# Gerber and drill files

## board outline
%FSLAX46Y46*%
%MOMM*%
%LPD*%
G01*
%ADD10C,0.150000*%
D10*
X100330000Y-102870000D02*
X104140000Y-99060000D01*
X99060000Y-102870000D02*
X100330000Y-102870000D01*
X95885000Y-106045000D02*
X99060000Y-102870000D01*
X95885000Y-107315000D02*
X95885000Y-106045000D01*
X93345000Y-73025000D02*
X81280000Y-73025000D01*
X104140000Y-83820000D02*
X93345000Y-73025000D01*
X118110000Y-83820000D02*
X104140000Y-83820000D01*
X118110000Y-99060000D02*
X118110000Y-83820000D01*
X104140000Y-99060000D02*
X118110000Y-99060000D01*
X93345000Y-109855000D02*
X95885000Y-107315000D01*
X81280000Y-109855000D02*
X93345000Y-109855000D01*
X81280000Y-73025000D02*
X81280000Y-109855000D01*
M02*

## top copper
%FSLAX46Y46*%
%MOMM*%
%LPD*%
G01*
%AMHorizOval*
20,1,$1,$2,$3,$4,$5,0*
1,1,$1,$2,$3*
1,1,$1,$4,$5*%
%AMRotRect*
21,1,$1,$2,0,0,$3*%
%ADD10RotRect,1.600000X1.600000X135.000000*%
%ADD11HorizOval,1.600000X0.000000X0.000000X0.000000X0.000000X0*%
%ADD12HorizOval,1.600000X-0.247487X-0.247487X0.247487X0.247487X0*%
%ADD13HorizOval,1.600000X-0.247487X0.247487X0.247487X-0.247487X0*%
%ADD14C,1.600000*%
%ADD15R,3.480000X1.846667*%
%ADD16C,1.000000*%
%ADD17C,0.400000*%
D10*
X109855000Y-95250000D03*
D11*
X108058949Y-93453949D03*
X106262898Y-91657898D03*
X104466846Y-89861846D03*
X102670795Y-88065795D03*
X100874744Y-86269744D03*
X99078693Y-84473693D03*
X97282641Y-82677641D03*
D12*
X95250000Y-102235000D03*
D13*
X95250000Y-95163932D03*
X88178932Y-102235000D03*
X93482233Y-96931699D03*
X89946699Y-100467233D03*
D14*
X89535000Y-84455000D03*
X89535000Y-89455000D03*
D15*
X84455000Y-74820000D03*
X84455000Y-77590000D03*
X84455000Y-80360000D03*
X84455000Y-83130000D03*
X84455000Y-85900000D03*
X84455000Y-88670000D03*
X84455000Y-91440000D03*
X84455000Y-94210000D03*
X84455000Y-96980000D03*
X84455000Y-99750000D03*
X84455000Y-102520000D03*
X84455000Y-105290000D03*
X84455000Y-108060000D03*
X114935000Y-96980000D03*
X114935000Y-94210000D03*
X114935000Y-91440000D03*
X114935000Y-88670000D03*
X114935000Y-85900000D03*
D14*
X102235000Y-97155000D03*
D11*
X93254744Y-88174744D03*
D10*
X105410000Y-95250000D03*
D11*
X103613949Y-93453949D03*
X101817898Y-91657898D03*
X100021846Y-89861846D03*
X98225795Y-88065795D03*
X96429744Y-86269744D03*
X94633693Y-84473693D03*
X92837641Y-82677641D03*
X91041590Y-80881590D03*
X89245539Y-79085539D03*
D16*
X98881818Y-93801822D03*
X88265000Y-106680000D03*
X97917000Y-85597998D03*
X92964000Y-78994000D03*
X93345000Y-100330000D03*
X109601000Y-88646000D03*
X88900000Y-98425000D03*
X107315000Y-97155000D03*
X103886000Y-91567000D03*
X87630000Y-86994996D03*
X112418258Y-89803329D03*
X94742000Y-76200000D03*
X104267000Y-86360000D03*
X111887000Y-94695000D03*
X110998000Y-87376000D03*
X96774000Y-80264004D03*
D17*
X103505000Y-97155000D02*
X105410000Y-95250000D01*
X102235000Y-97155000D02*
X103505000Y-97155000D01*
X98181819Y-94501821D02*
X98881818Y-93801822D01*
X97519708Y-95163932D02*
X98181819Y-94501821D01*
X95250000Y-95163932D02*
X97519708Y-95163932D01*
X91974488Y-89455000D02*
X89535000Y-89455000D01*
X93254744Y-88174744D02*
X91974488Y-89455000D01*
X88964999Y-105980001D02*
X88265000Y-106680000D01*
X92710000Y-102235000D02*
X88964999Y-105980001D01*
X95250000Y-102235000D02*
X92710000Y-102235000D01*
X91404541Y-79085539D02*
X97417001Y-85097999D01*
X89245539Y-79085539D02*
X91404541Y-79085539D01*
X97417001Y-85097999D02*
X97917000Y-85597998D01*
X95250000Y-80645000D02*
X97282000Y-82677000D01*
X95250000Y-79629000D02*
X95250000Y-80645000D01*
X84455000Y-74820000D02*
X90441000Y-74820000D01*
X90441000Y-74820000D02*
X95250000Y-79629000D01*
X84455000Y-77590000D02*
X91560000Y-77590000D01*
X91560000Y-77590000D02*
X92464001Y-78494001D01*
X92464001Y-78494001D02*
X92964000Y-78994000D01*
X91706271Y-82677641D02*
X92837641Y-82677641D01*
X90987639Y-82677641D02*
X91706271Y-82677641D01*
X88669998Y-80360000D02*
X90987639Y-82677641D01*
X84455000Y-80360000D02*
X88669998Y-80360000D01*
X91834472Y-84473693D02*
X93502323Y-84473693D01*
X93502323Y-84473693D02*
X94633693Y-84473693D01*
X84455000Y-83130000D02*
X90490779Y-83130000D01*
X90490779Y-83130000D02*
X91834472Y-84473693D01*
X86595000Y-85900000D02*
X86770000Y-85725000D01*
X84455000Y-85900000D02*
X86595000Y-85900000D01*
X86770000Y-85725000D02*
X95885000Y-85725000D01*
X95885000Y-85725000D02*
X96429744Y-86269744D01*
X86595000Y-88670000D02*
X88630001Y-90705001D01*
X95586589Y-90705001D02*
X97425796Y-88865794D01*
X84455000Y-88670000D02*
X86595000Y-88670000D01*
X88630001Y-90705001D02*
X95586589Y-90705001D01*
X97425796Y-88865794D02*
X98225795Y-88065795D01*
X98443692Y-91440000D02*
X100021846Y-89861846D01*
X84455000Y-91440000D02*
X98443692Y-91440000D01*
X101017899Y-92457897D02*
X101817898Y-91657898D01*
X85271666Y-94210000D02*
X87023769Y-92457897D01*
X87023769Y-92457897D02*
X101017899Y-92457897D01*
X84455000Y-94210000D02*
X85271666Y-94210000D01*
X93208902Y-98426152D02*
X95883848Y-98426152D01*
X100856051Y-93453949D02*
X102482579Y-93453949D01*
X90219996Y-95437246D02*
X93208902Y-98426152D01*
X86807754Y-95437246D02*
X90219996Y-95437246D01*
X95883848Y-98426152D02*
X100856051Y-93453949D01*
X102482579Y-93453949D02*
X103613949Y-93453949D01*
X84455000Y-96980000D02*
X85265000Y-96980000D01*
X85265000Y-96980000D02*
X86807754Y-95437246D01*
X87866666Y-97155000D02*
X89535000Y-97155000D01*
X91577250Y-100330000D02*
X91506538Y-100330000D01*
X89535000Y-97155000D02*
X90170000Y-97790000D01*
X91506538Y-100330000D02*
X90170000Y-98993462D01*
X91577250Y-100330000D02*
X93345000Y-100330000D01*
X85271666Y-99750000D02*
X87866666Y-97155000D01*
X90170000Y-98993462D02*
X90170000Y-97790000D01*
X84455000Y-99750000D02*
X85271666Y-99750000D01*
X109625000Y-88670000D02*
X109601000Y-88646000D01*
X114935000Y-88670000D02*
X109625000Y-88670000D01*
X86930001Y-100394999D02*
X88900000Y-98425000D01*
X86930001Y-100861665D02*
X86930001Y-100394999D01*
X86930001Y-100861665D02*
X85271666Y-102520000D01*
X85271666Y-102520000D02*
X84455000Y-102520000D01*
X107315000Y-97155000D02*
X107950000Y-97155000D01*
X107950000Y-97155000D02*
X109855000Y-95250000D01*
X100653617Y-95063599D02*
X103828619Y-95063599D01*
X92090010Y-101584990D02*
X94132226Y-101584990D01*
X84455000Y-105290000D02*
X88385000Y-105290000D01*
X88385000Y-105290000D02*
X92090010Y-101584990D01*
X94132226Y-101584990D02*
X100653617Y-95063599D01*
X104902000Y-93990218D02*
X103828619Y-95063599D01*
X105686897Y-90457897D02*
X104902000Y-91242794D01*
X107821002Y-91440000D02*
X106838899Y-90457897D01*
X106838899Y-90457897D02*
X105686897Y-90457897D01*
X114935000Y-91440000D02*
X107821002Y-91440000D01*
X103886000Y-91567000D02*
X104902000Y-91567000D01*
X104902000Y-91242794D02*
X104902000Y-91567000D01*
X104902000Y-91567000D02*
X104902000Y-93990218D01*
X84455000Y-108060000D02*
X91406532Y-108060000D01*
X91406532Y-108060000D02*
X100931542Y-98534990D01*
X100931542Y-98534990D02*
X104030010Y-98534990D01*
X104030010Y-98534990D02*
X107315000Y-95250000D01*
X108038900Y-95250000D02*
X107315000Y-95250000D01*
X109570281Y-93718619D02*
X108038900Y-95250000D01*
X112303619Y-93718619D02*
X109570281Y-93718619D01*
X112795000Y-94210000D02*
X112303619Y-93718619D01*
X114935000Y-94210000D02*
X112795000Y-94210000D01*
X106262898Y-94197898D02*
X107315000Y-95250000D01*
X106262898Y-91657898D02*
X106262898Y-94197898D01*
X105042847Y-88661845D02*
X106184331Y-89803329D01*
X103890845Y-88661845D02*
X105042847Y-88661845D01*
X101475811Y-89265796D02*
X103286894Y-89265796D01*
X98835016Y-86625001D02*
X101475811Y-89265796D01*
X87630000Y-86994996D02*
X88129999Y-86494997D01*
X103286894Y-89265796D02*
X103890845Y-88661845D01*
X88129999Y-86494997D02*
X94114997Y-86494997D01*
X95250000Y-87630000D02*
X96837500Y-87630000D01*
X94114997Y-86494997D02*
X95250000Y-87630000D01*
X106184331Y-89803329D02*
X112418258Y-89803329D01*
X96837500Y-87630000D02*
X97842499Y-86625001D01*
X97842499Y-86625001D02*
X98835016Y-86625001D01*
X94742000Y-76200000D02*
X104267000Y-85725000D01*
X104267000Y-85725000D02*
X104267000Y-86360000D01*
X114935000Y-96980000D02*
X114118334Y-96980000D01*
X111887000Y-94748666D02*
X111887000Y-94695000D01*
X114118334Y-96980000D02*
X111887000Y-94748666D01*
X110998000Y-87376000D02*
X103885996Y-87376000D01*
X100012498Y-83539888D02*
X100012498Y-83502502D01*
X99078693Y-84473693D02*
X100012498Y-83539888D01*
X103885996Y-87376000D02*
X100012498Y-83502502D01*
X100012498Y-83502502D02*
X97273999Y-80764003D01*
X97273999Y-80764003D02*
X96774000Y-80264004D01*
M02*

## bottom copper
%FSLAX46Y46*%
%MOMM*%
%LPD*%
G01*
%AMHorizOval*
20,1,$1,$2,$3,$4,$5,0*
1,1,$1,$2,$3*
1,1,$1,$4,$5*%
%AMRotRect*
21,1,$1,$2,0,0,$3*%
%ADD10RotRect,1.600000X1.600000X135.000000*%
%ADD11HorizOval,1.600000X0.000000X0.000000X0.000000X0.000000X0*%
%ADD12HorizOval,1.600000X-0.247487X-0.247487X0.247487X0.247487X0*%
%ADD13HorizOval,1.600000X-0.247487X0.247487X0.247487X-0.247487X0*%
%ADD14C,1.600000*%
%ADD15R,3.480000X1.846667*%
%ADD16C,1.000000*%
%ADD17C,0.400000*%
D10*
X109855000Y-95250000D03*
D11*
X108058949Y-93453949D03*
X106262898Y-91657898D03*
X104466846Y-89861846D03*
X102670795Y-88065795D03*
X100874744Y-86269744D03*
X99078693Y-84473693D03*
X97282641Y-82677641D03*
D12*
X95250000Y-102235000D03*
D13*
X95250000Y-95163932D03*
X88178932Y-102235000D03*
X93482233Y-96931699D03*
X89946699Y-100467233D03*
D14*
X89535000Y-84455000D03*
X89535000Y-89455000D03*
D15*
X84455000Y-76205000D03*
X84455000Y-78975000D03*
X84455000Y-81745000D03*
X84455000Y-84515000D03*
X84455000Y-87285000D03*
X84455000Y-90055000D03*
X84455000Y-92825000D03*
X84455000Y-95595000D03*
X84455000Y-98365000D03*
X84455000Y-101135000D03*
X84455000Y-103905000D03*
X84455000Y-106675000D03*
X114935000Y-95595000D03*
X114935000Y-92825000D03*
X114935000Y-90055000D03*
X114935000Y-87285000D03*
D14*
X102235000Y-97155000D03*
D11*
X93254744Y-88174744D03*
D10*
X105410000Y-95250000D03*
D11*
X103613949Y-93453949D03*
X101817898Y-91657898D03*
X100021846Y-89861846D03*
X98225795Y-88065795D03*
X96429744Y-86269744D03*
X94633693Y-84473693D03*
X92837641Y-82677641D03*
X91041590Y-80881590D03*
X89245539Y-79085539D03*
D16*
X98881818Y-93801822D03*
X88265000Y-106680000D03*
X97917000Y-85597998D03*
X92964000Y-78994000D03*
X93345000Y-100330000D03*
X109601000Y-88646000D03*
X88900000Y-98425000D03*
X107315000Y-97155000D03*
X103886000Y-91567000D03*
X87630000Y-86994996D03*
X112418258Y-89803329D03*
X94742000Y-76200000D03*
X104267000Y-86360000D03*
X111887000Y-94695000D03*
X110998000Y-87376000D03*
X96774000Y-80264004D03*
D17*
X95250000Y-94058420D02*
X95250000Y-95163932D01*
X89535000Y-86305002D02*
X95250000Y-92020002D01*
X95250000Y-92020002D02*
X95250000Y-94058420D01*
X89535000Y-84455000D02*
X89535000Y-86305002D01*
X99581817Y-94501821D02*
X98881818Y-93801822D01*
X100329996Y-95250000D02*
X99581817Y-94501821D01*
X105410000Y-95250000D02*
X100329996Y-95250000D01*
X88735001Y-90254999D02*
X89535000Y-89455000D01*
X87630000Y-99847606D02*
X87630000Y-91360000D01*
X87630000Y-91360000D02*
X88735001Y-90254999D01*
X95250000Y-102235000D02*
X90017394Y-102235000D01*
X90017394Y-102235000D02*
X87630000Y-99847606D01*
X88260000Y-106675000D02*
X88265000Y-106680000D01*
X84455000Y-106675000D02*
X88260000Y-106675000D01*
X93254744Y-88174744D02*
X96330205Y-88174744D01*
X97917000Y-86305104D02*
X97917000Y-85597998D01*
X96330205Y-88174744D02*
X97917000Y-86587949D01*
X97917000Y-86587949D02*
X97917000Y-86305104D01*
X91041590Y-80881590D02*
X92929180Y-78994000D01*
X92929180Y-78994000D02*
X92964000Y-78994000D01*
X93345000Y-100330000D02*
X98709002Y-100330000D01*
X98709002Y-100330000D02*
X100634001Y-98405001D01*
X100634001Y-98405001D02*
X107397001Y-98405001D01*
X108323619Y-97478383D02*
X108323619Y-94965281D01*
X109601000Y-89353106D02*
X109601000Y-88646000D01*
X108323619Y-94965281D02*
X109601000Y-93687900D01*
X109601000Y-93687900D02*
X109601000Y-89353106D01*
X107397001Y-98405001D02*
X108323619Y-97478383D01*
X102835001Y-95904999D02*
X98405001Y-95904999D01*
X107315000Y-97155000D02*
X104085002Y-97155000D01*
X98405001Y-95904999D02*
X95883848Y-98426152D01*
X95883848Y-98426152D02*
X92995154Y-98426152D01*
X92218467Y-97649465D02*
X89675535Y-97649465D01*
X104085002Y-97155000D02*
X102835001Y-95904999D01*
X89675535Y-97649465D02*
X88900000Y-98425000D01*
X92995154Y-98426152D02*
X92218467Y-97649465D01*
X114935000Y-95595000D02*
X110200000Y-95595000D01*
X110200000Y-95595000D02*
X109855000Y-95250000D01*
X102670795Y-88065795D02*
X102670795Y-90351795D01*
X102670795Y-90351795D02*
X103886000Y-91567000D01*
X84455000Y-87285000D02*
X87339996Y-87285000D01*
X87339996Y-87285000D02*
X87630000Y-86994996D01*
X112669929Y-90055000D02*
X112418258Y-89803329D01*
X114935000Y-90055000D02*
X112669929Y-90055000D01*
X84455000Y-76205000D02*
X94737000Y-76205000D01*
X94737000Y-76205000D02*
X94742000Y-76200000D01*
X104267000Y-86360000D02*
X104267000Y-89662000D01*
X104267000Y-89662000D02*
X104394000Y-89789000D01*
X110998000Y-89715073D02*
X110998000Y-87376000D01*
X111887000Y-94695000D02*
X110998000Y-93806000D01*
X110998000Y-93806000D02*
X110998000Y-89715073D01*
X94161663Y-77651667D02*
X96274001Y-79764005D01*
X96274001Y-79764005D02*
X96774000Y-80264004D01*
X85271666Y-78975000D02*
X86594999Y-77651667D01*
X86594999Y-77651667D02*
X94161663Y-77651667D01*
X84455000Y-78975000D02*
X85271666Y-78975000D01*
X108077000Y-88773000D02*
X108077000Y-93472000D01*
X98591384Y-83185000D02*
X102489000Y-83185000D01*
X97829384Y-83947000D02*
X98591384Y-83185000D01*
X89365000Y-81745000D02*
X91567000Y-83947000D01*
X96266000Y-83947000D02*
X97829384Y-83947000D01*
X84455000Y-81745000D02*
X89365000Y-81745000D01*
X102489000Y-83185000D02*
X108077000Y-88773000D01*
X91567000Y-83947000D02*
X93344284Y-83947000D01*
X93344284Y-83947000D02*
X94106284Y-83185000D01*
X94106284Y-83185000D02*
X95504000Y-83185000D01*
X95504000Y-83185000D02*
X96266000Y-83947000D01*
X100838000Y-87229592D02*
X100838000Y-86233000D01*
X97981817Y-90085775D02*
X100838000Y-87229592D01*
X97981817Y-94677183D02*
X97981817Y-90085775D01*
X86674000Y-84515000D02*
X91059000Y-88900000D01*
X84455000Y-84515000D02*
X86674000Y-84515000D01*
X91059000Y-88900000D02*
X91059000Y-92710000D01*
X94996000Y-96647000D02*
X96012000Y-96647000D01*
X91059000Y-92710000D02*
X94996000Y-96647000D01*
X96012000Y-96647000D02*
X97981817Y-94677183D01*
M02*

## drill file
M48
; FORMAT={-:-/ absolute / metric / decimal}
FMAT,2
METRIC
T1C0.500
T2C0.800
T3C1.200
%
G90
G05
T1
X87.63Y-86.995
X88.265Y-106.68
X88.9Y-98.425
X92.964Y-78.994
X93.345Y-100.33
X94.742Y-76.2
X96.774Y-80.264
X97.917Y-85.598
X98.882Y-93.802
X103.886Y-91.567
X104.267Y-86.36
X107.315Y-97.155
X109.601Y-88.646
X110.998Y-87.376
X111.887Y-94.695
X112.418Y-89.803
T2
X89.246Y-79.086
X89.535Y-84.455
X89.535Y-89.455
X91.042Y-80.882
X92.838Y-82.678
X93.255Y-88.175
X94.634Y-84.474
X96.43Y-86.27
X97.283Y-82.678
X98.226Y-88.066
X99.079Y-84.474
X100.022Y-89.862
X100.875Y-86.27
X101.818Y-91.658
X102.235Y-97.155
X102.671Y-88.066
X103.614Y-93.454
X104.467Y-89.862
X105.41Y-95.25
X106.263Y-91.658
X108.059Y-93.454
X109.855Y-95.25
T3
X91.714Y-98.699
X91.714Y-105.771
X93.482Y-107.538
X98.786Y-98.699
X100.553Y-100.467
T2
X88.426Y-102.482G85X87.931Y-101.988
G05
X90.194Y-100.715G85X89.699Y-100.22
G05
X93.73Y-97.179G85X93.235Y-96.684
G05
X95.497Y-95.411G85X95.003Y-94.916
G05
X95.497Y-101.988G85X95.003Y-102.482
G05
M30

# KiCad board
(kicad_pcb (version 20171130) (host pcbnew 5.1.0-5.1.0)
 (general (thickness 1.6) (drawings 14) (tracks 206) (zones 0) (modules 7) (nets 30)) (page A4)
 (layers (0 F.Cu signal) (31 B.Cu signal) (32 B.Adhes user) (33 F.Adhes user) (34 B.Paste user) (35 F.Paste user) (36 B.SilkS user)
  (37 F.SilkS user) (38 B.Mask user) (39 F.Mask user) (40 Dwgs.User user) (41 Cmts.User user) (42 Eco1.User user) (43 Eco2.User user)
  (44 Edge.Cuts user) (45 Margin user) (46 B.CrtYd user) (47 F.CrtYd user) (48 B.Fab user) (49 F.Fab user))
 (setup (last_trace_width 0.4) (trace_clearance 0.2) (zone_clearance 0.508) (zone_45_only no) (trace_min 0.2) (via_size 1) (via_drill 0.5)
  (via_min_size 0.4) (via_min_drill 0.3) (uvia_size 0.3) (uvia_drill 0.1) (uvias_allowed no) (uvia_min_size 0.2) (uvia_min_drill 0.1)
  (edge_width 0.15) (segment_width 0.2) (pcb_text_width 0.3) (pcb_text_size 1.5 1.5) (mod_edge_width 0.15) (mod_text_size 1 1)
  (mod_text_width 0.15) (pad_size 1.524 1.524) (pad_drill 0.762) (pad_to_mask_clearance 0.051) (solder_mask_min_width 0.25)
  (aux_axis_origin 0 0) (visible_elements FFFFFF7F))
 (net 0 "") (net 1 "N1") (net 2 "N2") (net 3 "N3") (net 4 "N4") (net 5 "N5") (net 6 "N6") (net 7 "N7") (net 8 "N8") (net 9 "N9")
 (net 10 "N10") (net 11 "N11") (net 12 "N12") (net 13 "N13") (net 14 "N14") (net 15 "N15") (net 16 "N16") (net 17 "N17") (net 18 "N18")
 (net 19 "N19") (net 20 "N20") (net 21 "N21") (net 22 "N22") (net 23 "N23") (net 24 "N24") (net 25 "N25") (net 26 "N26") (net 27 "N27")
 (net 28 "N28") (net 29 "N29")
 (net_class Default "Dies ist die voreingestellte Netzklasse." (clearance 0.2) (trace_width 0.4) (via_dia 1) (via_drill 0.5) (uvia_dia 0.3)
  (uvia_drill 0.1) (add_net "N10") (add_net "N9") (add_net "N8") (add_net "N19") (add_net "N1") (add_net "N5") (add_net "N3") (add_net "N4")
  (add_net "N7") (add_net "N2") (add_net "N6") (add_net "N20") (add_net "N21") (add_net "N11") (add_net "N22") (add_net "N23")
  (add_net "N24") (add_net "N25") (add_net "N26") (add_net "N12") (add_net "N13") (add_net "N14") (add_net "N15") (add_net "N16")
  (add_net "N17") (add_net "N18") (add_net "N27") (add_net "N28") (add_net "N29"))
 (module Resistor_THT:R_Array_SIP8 (layer F.Cu) (at 109.855 95.25 135)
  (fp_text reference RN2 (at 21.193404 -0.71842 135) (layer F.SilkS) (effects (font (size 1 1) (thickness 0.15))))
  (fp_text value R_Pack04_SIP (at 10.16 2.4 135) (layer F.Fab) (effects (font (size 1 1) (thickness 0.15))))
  (pad 1 thru_hole rect (at 0 0 135) (size 1.6 1.6) (drill 0.8) (layers *.Cu *.Mask) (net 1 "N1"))
  (pad 2 thru_hole oval (at 2.54 0 135) (size 1.6 1.6) (drill 0.8) (layers *.Cu *.Mask) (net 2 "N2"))
  (pad 3 thru_hole oval (at 5.08 0 135) (size 1.6 1.6) (drill 0.8) (layers *.Cu *.Mask) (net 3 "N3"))
  (pad 4 thru_hole oval (at 7.62 0 135) (size 1.6 1.6) (drill 0.8) (layers *.Cu *.Mask) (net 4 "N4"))
  (pad 5 thru_hole oval (at 10.16 0 135) (size 1.6 1.6) (drill 0.8) (layers *.Cu *.Mask) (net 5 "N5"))
  (pad 6 thru_hole oval (at 12.7 0 135) (size 1.6 1.6) (drill 0.8) (layers *.Cu *.Mask) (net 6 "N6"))
  (pad 7 thru_hole oval (at 15.24 0 135) (size 1.6 1.6) (drill 0.8) (layers *.Cu *.Mask) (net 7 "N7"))
  (pad 8 thru_hole oval (at 17.78 0 135) (size 1.6 1.6) (drill 0.8) (layers *.Cu *.Mask) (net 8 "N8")))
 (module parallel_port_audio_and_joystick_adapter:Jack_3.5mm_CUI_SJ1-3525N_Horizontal (layer F.Cu) (at 95.25 102.235 225)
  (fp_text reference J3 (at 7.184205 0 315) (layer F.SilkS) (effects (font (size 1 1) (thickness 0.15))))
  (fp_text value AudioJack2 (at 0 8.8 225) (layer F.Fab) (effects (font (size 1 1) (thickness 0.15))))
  (pad S thru_hole oval (at 0 0 225) (size 2.3 1.6) (drill oval 1.5 0.8) (layers *.Cu *.Mask) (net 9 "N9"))
  (pad T thru_hole oval (at -5 5 225) (size 1.6 2.3) (drill oval 0.8 1.5) (layers *.Cu *.Mask) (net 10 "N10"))
  (pad R thru_hole oval (at 5 5 225) (size 1.6 2.3) (drill oval 0.8 1.5) (layers *.Cu *.Mask))
  (pad TN thru_hole oval (at -2.5 5 225) (size 1.6 2.3) (drill oval 0.8 1.5) (layers *.Cu *.Mask))
  (pad RN thru_hole oval (at 2.5 5 225) (size 1.6 2.3) (drill oval 0.8 1.5) (layers *.Cu *.Mask))
  (pad "" np_thru_hole circle (at 0 5 225) (size 1.2 1.2) (drill 1.2) (layers *.Cu *.Mask))
  (pad "" np_thru_hole circle (at -5 0 225) (size 1.2 1.2) (drill 1.2) (layers *.Cu *.Mask))
  (pad "" np_thru_hole circle (at 5 0 225) (size 1.2 1.2) (drill 1.2) (layers *.Cu *.Mask))
  (pad "" np_thru_hole circle (at 5 -2.5 225) (size 1.2 1.2) (drill 1.2) (layers *.Cu *.Mask))
  (pad "" np_thru_hole circle (at -5 -2.5 225) (size 1.2 1.2) (drill 1.2) (layers *.Cu *.Mask)))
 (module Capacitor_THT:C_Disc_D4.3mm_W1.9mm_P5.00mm (layer F.Cu) (at 89.535 84.455 270)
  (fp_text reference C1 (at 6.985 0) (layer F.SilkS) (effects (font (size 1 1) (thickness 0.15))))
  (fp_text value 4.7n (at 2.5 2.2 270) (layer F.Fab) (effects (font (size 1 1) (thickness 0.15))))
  (pad 1 thru_hole circle (at 0 0 270) (size 1.6 1.6) (drill 0.8) (layers *.Cu *.Mask) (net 10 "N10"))
  (pad 2 thru_hole circle (at 5 0 270) (size 1.6 1.6) (drill 0.8) (layers *.Cu *.Mask) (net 9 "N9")))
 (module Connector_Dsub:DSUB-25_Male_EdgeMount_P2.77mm (layer F.Cu) (at 84.455 91.44 270)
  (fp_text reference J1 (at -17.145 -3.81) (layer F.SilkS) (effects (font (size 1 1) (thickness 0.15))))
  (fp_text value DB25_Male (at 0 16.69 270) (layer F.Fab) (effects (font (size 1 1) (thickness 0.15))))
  (pad 1 smd rect (at -16.62 0 270) (size 1.846667 3.48) (layers F.Cu F.Paste F.Mask) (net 8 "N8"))
  (pad 2 smd rect (at -13.85 0 270) (size 1.846667 3.48) (layers F.Cu F.Paste F.Mask) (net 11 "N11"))
  (pad 3 smd rect (at -11.08 0 270) (size 1.846667 3.48) (layers F.Cu F.Paste F.Mask) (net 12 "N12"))
  (pad 4 smd rect (at -8.31 0 270) (size 1.846667 3.48) (layers F.Cu F.Paste F.Mask) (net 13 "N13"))
  (pad 5 smd rect (at -5.54 0 270) (size 1.846667 3.48) (layers F.Cu F.Paste F.Mask) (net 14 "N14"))
  (pad 6 smd rect (at -2.77 0 270) (size 1.846667 3.48) (layers F.Cu F.Paste F.Mask) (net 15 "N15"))
  (pad 7 smd rect (at 0 0 270) (size 1.846667 3.48) (layers F.Cu F.Paste F.Mask) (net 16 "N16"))
  (pad 8 smd rect (at 2.77 0 270) (size 1.846667 3.48) (layers F.Cu F.Paste F.Mask) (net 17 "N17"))
  (pad 9 smd rect (at 5.54 0 270) (size 1.846667 3.48) (layers F.Cu F.Paste F.Mask) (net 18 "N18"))
  (pad 10 smd rect (at 8.31 0 270) (size 1.846667 3.48) (layers F.Cu F.Paste F.Mask) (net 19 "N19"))
  (pad 11 smd rect (at 11.08 0 270) (size 1.846667 3.48) (layers F.Cu F.Paste F.Mask) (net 1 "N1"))
  (pad 12 smd rect (at 13.85 0 270) (size 1.846667 3.48) (layers F.Cu F.Paste F.Mask) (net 5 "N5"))
  (pad 13 smd rect (at 16.62 0 270) (size 1.846667 3.48) (layers F.Cu F.Paste F.Mask) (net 3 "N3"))
  (pad 14 smd rect (at -15.235 0 270) (size 1.846667 3.48) (layers B.Cu B.Paste B.Mask) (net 4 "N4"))
  (pad 15 smd rect (at -12.465 0 270) (size 1.846667 3.48) (layers B.Cu B.Paste B.Mask) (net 7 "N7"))
  (pad 16 smd rect (at -9.695 0 270) (size 1.846667 3.48) (layers B.Cu B.Paste B.Mask) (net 2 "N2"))
  (pad 17 smd rect (at -6.925 0 270) (size 1.846667 3.48) (layers B.Cu B.Paste B.Mask) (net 6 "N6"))
  (pad 18 smd rect (at -4.155 0 270) (size 1.846667 3.48) (layers B.Cu B.Paste B.Mask) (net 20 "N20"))
  (pad 19 smd rect (at -1.385 0 270) (size 1.846667 3.48) (layers B.Cu B.Paste B.Mask) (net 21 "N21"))
  (pad 20 smd rect (at 1.385 0 270) (size 1.846667 3.48) (layers B.Cu B.Paste B.Mask) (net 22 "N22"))
  (pad 21 smd rect (at 4.155 0 270) (size 1.846667 3.48) (layers B.Cu B.Paste B.Mask) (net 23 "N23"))
  (pad 22 smd rect (at 6.925 0 270) (size 1.846667 3.48) (layers B.Cu B.Paste B.Mask) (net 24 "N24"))
  (pad 23 smd rect (at 9.695 0 270) (size 1.846667 3.48) (layers B.Cu B.Paste B.Mask) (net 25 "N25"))
  (pad 24 smd rect (at 12.465 0 270) (size 1.846667 3.48) (layers B.Cu B.Paste B.Mask) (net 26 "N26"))
  (pad 25 smd rect (at 15.235 0 270) (size 1.846667 3.48) (layers B.Cu B.Paste B.Mask) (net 9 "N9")))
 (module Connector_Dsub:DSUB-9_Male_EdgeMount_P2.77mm (layer F.Cu) (at 114.935 91.44 90)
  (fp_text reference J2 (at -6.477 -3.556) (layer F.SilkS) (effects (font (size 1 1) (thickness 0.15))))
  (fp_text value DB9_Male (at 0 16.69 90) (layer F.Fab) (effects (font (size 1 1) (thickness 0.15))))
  (pad 1 smd rect (at -5.54 0 90) (size 1.846667 3.48) (layers F.Cu F.Paste F.Mask) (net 7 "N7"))
  (pad 2 smd rect (at -2.77 0 90) (size 1.846667 3.48) (layers F.Cu F.Paste F.Mask) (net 3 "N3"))
  (pad 3 smd rect (at 0 0 90) (size 1.846667 3.48) (layers F.Cu F.Paste F.Mask) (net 5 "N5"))
  (pad 4 smd rect (at 2.77 0 90) (size 1.846667 3.48) (layers F.Cu F.Paste F.Mask) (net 19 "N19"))
  (pad 5 smd rect (at 5.54 0 90) (size 1.846667 3.48) (layers F.Cu F.Paste F.Mask) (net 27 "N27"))
  (pad 6 smd rect (at -4.155 0 90) (size 1.846667 3.48) (layers B.Cu B.Paste B.Mask) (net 1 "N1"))
  (pad 7 smd rect (at -1.385 0 90) (size 1.846667 3.48) (layers B.Cu B.Paste B.Mask) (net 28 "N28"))
  (pad 8 smd rect (at 1.385 0 90) (size 1.846667 3.48) (layers B.Cu B.Paste B.Mask) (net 20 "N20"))
  (pad 9 smd rect (at 4.155 0 90) (size 1.846667 3.48) (layers B.Cu B.Paste B.Mask) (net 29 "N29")))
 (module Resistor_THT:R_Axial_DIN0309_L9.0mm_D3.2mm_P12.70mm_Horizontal (layer F.Cu) (at 102.235 97.155 135)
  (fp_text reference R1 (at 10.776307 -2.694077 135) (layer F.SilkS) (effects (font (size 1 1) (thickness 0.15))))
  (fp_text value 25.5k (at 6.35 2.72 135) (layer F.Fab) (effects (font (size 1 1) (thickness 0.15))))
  (pad 1 thru_hole circle (at 0 0 135) (size 1.6 1.6) (drill 0.8) (layers *.Cu *.Mask) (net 10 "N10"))
  (pad 2 thru_hole oval (at 12.7 0 135) (size 1.6 1.6) (drill 0.8) (layers *.Cu *.Mask) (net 9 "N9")))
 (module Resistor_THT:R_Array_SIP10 (layer F.Cu) (at 105.41 95.25 135)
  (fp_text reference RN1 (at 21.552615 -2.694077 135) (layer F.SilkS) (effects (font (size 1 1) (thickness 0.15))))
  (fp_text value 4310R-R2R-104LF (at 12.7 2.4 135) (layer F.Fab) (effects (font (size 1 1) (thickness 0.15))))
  (pad 1 thru_hole rect (at 0 0 135) (size 1.6 1.6) (drill 0.8) (layers *.Cu *.Mask) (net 10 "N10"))
  (pad 2 thru_hole oval (at 2.54 0 135) (size 1.6 1.6) (drill 0.8) (layers *.Cu *.Mask) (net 18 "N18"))
  (pad 3 thru_hole oval (at 5.079999 0 135) (size 1.6 1.6) (drill 0.8) (layers *.Cu *.Mask) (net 17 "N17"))
  (pad 4 thru_hole oval (at 7.62 0 135) (size 1.6 1.6) (drill 0.8) (layers *.Cu *.Mask) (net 16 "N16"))
  (pad 5 thru_hole oval (at 10.16 0 135) (size 1.6 1.6) (drill 0.8) (layers *.Cu *.Mask) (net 15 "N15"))
  (pad 6 thru_hole oval (at 12.7 0 135) (size 1.6 1.6) (drill 0.8) (layers *.Cu *.Mask) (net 14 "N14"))
  (pad 7 thru_hole oval (at 15.24 0 135) (size 1.6 1.6) (drill 0.8) (layers *.Cu *.Mask) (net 13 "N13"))
  (pad 8 thru_hole oval (at 17.780001 0 135) (size 1.6 1.6) (drill 0.8) (layers *.Cu *.Mask) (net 12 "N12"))
  (pad 9 thru_hole oval (at 20.32 0 135) (size 1.6 1.6) (drill 0.8) (layers *.Cu *.Mask) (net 11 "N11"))
  (pad 10 thru_hole oval (at 22.86 0 135) (size 1.6 1.6) (drill 0.8) (layers *.Cu *.Mask) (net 9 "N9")))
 (gr_line (start 100.33 102.87) (end 104.14 99.06) (layer Edge.Cuts) (width 0.15))
 (gr_line (start 99.06 102.87) (end 100.33 102.87) (layer Edge.Cuts) (width 0.15))
 (gr_line (start 95.885 106.045) (end 99.06 102.87) (layer Edge.Cuts) (width 0.15))
 (gr_line (start 95.885 107.315) (end 95.885 106.045) (layer Edge.Cuts) (width 0.15))
 (gr_line (start 93.345 73.025) (end 81.28 73.025) (layer Edge.Cuts) (width 0.15))
 (gr_line (start 104.14 83.82) (end 93.345 73.025) (layer Edge.Cuts) (width 0.15))
 (gr_line (start 118.11 83.82) (end 104.14 83.82) (layer Edge.Cuts) (width 0.15))
 (gr_line (start 118.11 99.06) (end 118.11 83.82) (layer Edge.Cuts) (width 0.15))
 (gr_line (start 104.14 99.06) (end 118.11 99.06) (layer Edge.Cuts) (width 0.15))
 (gr_line (start 93.345 109.855) (end 95.885 107.315) (layer Edge.Cuts) (width 0.15))
 (gr_line (start 81.28 109.855) (end 93.345 109.855) (layer Edge.Cuts) (width 0.15))
 (gr_line (start 81.28 73.025) (end 81.28 109.855) (layer Edge.Cuts) (width 0.15))
 (segment (start 103.505 97.155) (end 105.41 95.25) (width 0.4) (layer F.Cu) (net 10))
 (segment (start 102.235 97.155) (end 103.505 97.155) (width 0.4) (layer F.Cu) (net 10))
 (segment (start 95.25 94.05842) (end 95.25 95.163932) (width 0.4) (layer B.Cu) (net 10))
 (segment (start 89.535 86.305002) (end 95.25 92.020002) (width 0.4) (layer B.Cu) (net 10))
 (segment (start 95.25 92.020002) (end 95.25 94.05842) (width 0.4) (layer B.Cu) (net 10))
 (segment (start 89.535 84.455) (end 89.535 86.305002) (width 0.4) (layer B.Cu) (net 10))
 (via (at 98.881818 93.801822) (size 1) (drill 0.5) (layers F.Cu B.Cu) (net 10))
 (segment (start 98.181819 94.501821) (end 98.881818 93.801822) (width 0.4) (layer F.Cu) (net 10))
 (segment (start 99.581817 94.501821) (end 98.881818 93.801822) (width 0.4) (layer B.Cu) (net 10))
 (segment (start 97.519708 95.163932) (end 98.181819 94.501821) (width 0.4) (layer F.Cu) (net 10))
 (segment (start 95.25 95.163932) (end 97.519708 95.163932) (width 0.4) (layer F.Cu) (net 10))
 (segment (start 100.329996 95.25) (end 99.581817 94.501821) (width 0.4) (layer B.Cu) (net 10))
 (segment (start 105.41 95.25) (end 100.329996 95.25) (width 0.4) (layer B.Cu) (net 10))
 (segment (start 91.974488 89.455) (end 89.535 89.455) (width 0.4) (layer F.Cu) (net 9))
 (segment (start 93.254744 88.174744) (end 91.974488 89.455) (width 0.4) (layer F.Cu) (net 9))
 (segment (start 88.735001 90.254999) (end 89.535 89.455) (width 0.4) (layer B.Cu) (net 9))
 (segment (start 87.63 99.847606) (end 87.63 91.36) (width 0.4) (layer B.Cu) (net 9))
 (segment (start 87.63 91.36) (end 88.735001 90.254999) (width 0.4) (layer B.Cu) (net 9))
 (segment (start 95.25 102.235) (end 90.017394 102.235) (width 0.4) (layer B.Cu) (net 9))
 (segment (start 90.017394 102.235) (end 87.63 99.847606) (width 0.4) (layer B.Cu) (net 9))
 (segment (start 88.964999 105.980001) (end 88.265 106.68) (width 0.4) (layer F.Cu) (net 9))
 (segment (start 92.71 102.235) (end 88.964999 105.980001) (width 0.4) (layer F.Cu) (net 9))
 (segment (start 95.25 102.235) (end 92.71 102.235) (width 0.4) (layer F.Cu) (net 9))
 (segment (start 88.26 106.675) (end 88.265 106.68) (width 0.4) (layer B.Cu) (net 9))
 (via (at 88.265 106.68) (size 1) (drill 0.5) (layers F.Cu B.Cu) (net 9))
 (segment (start 84.455 106.675) (end 88.26 106.675) (width 0.4) (layer B.Cu) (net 9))
 (segment (start 93.254744 88.174744) (end 96.330205 88.174744) (width 0.4) (layer B.Cu) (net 9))
 (via (at 97.917 85.597998) (size 1) (drill 0.5) (layers F.Cu B.Cu) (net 9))
 (segment (start 91.404541 79.085539) (end 97.417001 85.097999) (width 0.4) (layer F.Cu) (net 9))
 (segment (start 97.917 86.305104) (end 97.917 85.597998) (width 0.4) (layer B.Cu) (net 9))
 (segment (start 96.330205 88.174744) (end 97.917 86.587949) (width 0.4) (layer B.Cu) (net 9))
 (segment (start 89.245539 79.085539) (end 91.404541 79.085539) (width 0.4) (layer F.Cu) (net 9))
 (segment (start 97.917 86.587949) (end 97.917 86.305104) (width 0.4) (layer B.Cu) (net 9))
 (segment (start 97.417001 85.097999) (end 97.917 85.597998) (width 0.4) (layer F.Cu) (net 9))
 (segment (start 95.25 80.645) (end 97.282 82.677) (width 0.4) (layer F.Cu) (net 8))
 (segment (start 95.25 79.629) (end 95.25 80.645) (width 0.4) (layer F.Cu) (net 8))
 (segment (start 84.455 74.82) (end 90.441 74.82) (width 0.4) (layer F.Cu) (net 8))
 (segment (start 90.441 74.82) (end 95.25 79.629) (width 0.4) (layer F.Cu) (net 8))
 (segment (start 91.04159 80.88159) (end 92.92918 78.994) (width 0.4) (layer B.Cu) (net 11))
 (via (at 92.964 78.994) (size 1) (drill 0.5) (layers F.Cu B.Cu) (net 11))
 (segment (start 92.92918 78.994) (end 92.964 78.994) (width 0.4) (layer B.Cu) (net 11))
 (segment (start 84.455 77.59) (end 91.56 77.59) (width 0.4) (layer F.Cu) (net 11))
 (segment (start 91.56 77.59) (end 92.464001 78.494001) (width 0.4) (layer F.Cu) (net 11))
 (segment (start 92.464001 78.494001) (end 92.964 78.994) (width 0.4) (layer F.Cu) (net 11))
 (segment (start 91.706271 82.677641) (end 92.837641 82.677641) (width 0.4) (layer F.Cu) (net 12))
 (segment (start 90.987639 82.677641) (end 91.706271 82.677641) (width 0.4) (layer F.Cu) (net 12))
 (segment (start 88.669998 80.36) (end 90.987639 82.677641) (width 0.4) (layer F.Cu) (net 12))
 (segment (start 84.455 80.36) (end 88.669998 80.36) (width 0.4) (layer F.Cu) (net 12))
 (segment (start 91.834472 84.473693) (end 93.502323 84.473693) (width 0.4) (layer F.Cu) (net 13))
 (segment (start 93.502323 84.473693) (end 94.633693 84.473693) (width 0.4) (layer F.Cu) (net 13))
 (segment (start 84.455 83.13) (end 90.490779 83.13) (width 0.4) (layer F.Cu) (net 13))
 (segment (start 90.490779 83.13) (end 91.834472 84.473693) (width 0.4) (layer F.Cu) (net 13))
 (segment (start 86.595 85.9) (end 86.77 85.725) (width 0.4) (layer F.Cu) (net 14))
 (segment (start 84.455 85.9) (end 86.595 85.9) (width 0.4) (layer F.Cu) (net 14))
 (segment (start 86.77 85.725) (end 95.885 85.725) (width 0.4) (layer F.Cu) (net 14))
 (segment (start 95.885 85.725) (end 96.429744 86.269744) (width 0.4) (layer F.Cu) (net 14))
 (segment (start 86.595 88.67) (end 88.630001 90.705001) (width 0.4) (layer F.Cu) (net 15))
 (segment (start 95.586589 90.705001) (end 97.425796 88.865794) (width 0.4) (layer F.Cu) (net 15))
 (segment (start 84.455 88.67) (end 86.595 88.67) (width 0.4) (layer F.Cu) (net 15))
 (segment (start 88.630001 90.705001) (end 95.586589 90.705001) (width 0.4) (layer F.Cu) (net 15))
 (segment (start 97.425796 88.865794) (end 98.225795 88.065795) (width 0.4) (layer F.Cu) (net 15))
 (segment (start 98.443692 91.44) (end 100.021846 89.861846) (width 0.4) (layer F.Cu) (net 16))
 (segment (start 84.455 91.44) (end 98.443692 91.44) (width 0.4) (layer F.Cu) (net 16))
 (segment (start 101.017899 92.457897) (end 101.817898 91.657898) (width 0.4) (layer F.Cu) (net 17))
 (segment (start 85.271666 94.21) (end 87.023769 92.457897) (width 0.4) (layer F.Cu) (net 17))
 (segment (start 87.023769 92.457897) (end 101.017899 92.457897) (width 0.4) (layer F.Cu) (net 17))
 (segment (start 84.455 94.21) (end 85.271666 94.21) (width 0.4) (layer F.Cu) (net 17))
 (segment (start 93.208902 98.426152) (end 95.883848 98.426152) (width 0.4) (layer F.Cu) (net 18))
 (segment (start 100.856051 93.453949) (end 102.482579 93.453949) (width 0.4) (layer F.Cu) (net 18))
 (segment (start 90.219996 95.437246) (end 93.208902 98.426152) (width 0.4) (layer F.Cu) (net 18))
 (segment (start 86.807754 95.437246) (end 90.219996 95.437246) (width 0.4) (layer F.Cu) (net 18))
 (segment (start 95.883848 98.426152) (end 100.856051 93.453949) (width 0.4) (layer F.Cu) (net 18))
 (segment (start 102.482579 93.453949) (end 103.613949 93.453949) (width 0.4) (layer F.Cu) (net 18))
 (segment (start 84.455 96.98) (end 85.265 96.98) (width 0.4) (layer F.Cu) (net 18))
 (segment (start 85.265 96.98) (end 86.807754 95.437246) (width 0.4) (layer F.Cu) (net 18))
 (via (at 93.345 100.33) (size 1) (drill 0.5) (layers F.Cu B.Cu) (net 19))
 (segment (start 87.866666 97.155) (end 89.535 97.155) (width 0.4) (layer F.Cu) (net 19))
 (segment (start 91.57725 100.33) (end 91.506538 100.33) (width 0.4) (layer F.Cu) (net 19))
 (segment (start 89.535 97.155) (end 90.17 97.79) (width 0.4) (layer F.Cu) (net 19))
 (segment (start 91.506538 100.33) (end 90.17 98.993462) (width 0.4) (layer F.Cu) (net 19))
 (segment (start 91.57725 100.33) (end 93.345 100.33) (width 0.4) (layer F.Cu) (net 19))
 (segment (start 85.271666 99.75) (end 87.866666 97.155) (width 0.4) (layer F.Cu) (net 19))
 (segment (start 90.17 98.993462) (end 90.17 97.79) (width 0.4) (layer F.Cu) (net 19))
 (segment (start 84.455 99.75) (end 85.271666 99.75) (width 0.4) (layer F.Cu) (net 19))
 (segment (start 93.345 100.33) (end 98.709002 100.33) (width 0.4) (layer B.Cu) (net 19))
 (segment (start 98.709002 100.33) (end 100.634001 98.405001) (width 0.4) (layer B.Cu) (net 19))
 (segment (start 100.634001 98.405001) (end 107.397001 98.405001) (width 0.4) (layer B.Cu) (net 19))
 (segment (start 108.323619 97.478383) (end 108.323619 94.965281) (width 0.4) (layer B.Cu) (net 19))
 (segment (start 109.601 89.353106) (end 109.601 88.646) (width 0.4) (layer B.Cu) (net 19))
 (segment (start 109.625 88.67) (end 109.601 88.646) (width 0.4) (layer F.Cu) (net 19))
 (segment (start 108.323619 94.965281) (end 109.601 93.6879) (width 0.4) (layer B.Cu) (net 19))
 (segment (start 109.601 93.6879) (end 109.601 89.353106) (width 0.4) (layer B.Cu) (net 19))
 (via (at 109.601 88.646) (size 1) (drill 0.5) (layers F.Cu B.Cu) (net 19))
 (segment (start 107.397001 98.405001) (end 108.323619 97.478383) (width 0.4) (layer B.Cu) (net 19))
 (segment (start 114.935 88.67) (end 109.625 88.67) (width 0.4) (layer F.Cu) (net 19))
 (segment (start 102.835001 95.904999) (end 98.405001 95.904999) (width 0.4) (layer B.Cu) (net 1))
 (segment (start 107.315 97.155) (end 104.085002 97.155) (width 0.4) (layer B.Cu) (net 1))
 (segment (start 98.405001 95.904999) (end 95.883848 98.426152) (width 0.4) (layer B.Cu) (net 1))
 (segment (start 95.883848 98.426152) (end 92.995154 98.426152) (width 0.4) (layer B.Cu) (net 1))
 (segment (start 92.218467 97.649465) (end 89.675535 97.649465) (width 0.4) (layer B.Cu) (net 1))
 (segment (start 104.085002 97.155) (end 102.835001 95.904999) (width 0.4) (layer B.Cu) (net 1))
 (segment (start 89.675535 97.649465) (end 88.9 98.425) (width 0.4) (layer B.Cu) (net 1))
 (segment (start 92.995154 98.426152) (end 92.218467 97.649465) (width 0.4) (layer B.Cu) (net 1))
 (segment (start 86.930001 100.394999) (end 88.9 98.425) (width 0.4) (layer F.Cu) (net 1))
 (segment (start 86.930001 100.861665) (end 86.930001 100.394999) (width 0.4) (layer F.Cu) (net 1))
 (via (at 88.9 98.425) (size 1) (drill 0.5) (layers F.Cu B.Cu) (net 1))
 (segment (start 86.930001 100.861665) (end 85.271666 102.52) (width 0.4) (layer F.Cu) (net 1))
 (segment (start 85.271666 102.52) (end 84.455 102.52) (width 0.4) (layer F.Cu) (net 1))
 (via (at 107.315 97.155) (size 1) (drill 0.5) (layers F.Cu B.Cu) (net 1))
 (segment (start 107.315 97.155) (end 107.95 97.155) (width 0.4) (layer F.Cu) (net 1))
 (segment (start 107.95 97.155) (end 109.855 95.25) (width 0.4) (layer F.Cu) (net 1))
 (segment (start 114.935 95.595) (end 110.2 95.595) (width 0.4) (layer B.Cu) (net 1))
 (segment (start 110.2 95.595) (end 109.855 95.25) (width 0.4) (layer B.Cu) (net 1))
 (segment (start 100.653617 95.063599) (end 103.828619 95.063599) (width 0.4) (layer F.Cu) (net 5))
 (segment (start 92.09001 101.58499) (end 94.132226 101.58499) (width 0.4) (layer F.Cu) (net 5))
 (segment (start 84.455 105.29) (end 88.385 105.29) (width 0.4) (layer F.Cu) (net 5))
 (segment (start 88.385 105.29) (end 92.09001 101.58499) (width 0.4) (layer F.Cu) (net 5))
 (segment (start 94.132226 101.58499) (end 100.653617 95.063599) (width 0.4) (layer F.Cu) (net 5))
 (segment (start 104.902 93.990218) (end 103.828619 95.063599) (width 0.4) (layer F.Cu) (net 5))
 (segment (start 105.686897 90.457897) (end 104.902 91.242794) (width 0.4) (layer F.Cu) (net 5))
 (segment (start 107.821002 91.44) (end 106.838899 90.457897) (width 0.4) (layer F.Cu) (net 5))
 (segment (start 106.838899 90.457897) (end 105.686897 90.457897) (width 0.4) (layer F.Cu) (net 5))
 (segment (start 114.935 91.44) (end 107.821002 91.44) (width 0.4) (layer F.Cu) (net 5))
 (via (at 103.886 91.567) (size 1) (drill 0.5) (layers F.Cu B.Cu) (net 5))
 (segment (start 102.670795 88.065795) (end 102.670795 90.351795) (width 0.4) (layer B.Cu) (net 5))
 (segment (start 102.670795 90.351795) (end 103.886 91.567) (width 0.4) (layer B.Cu) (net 5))
 (segment (start 103.886 91.567) (end 104.902 91.567) (width 0.4) (layer F.Cu) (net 5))
 (segment (start 104.902 91.242794) (end 104.902 91.567) (width 0.4) (layer F.Cu) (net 5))
 (segment (start 104.902 91.567) (end 104.902 93.990218) (width 0.4) (layer F.Cu) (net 5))
 (segment (start 84.455 108.06) (end 91.406532 108.06) (width 0.4) (layer F.Cu) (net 3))
 (segment (start 91.406532 108.06) (end 100.931542 98.53499) (width 0.4) (layer F.Cu) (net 3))
 (segment (start 100.931542 98.53499) (end 104.03001 98.53499) (width 0.4) (layer F.Cu) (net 3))
 (segment (start 104.03001 98.53499) (end 107.315 95.25) (width 0.4) (layer F.Cu) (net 3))
 (segment (start 108.0389 95.25) (end 107.315 95.25) (width 0.4) (layer F.Cu) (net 3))
 (segment (start 109.570281 93.718619) (end 108.0389 95.25) (width 0.4) (layer F.Cu) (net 3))
 (segment (start 112.303619 93.718619) (end 109.570281 93.718619) (width 0.4) (layer F.Cu) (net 3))
 (segment (start 112.795 94.21) (end 112.303619 93.718619) (width 0.4) (layer F.Cu) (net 3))
 (segment (start 114.935 94.21) (end 112.795 94.21) (width 0.4) (layer F.Cu) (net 3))
 (segment (start 106.262898 94.197898) (end 107.315 95.25) (width 0.4) (layer F.Cu) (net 3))
 (segment (start 106.262898 91.657898) (end 106.262898 94.197898) (width 0.4) (layer F.Cu) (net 3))
 (via (at 87.63 86.994996) (size 1) (drill 0.5) (layers F.Cu B.Cu) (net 20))
 (segment (start 84.455 87.285) (end 87.339996 87.285) (width 0.4) (layer B.Cu) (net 20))
 (segment (start 87.339996 87.285) (end 87.63 86.994996) (width 0.4) (layer B.Cu) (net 20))
 (via (at 112.418258 89.803329) (size 1) (drill 0.5) (layers F.Cu B.Cu) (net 20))
 (segment (start 112.669929 90.055) (end 112.418258 89.803329) (width 0.4) (layer B.Cu) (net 20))
 (segment (start 114.935 90.055) (end 112.669929 90.055) (width 0.4) (layer B.Cu) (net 20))
 (segment (start 105.042847 88.661845) (end 106.184331 89.803329) (width 0.4) (layer F.Cu) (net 20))
 (segment (start 103.890845 88.661845) (end 105.042847 88.661845) (width 0.4) (layer F.Cu) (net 20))
 (segment (start 101.475811 89.265796) (end 103.286894 89.265796) (width 0.4) (layer F.Cu) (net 20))
 (segment (start 98.835016 86.625001) (end 101.475811 89.265796) (width 0.4) (layer F.Cu) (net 20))
 (segment (start 87.63 86.994996) (end 88.129999 86.494997) (width 0.4) (layer F.Cu) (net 20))
 (segment (start 103.286894 89.265796) (end 103.890845 88.661845) (width 0.4) (layer F.Cu) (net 20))
 (segment (start 88.129999 86.494997) (end 94.114997 86.494997) (width 0.4) (layer F.Cu) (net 20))
 (segment (start 95.25 87.63) (end 96.8375 87.63) (width 0.4) (layer F.Cu) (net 20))
 (segment (start 94.114997 86.494997) (end 95.25 87.63) (width 0.4) (layer F.Cu) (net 20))
 (segment (start 106.184331 89.803329) (end 112.418258 89.803329) (width 0.4) (layer F.Cu) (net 20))
 (segment (start 96.8375 87.63) (end 97.842499 86.625001) (width 0.4) (layer F.Cu) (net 20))
 (segment (start 97.842499 86.625001) (end 98.835016 86.625001) (width 0.4) (layer F.Cu) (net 20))
 (via (at 94.742 76.2) (size 1) (drill 0.5) (layers F.Cu B.Cu) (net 4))
 (segment (start 84.455 76.205) (end 94.737 76.205) (width 0.4) (layer B.Cu) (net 4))
 (segment (start 94.737 76.205) (end 94.742 76.2) (width 0.4) (layer B.Cu) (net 4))
 (segment (start 94.742 76.2) (end 104.267 85.725) (width 0.4) (layer F.Cu) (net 4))
 (via (at 104.267 86.36) (size 1) (drill 0.5) (layers F.Cu B.Cu) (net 4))
 (segment (start 104.267 85.725) (end 104.267 86.36) (width 0.4) (layer F.Cu) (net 4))
 (segment (start 104.267 86.36) (end 104.267 89.662) (width 0.4) (layer B.Cu) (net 4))
 (segment (start 104.267 89.662) (end 104.394 89.789) (width 0.4) (layer B.Cu) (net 4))
 (via (at 111.887 94.695) (size 1) (drill 0.5) (layers F.Cu B.Cu) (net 7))
 (segment (start 114.935 96.98) (end 114.118334 96.98) (width 0.4) (layer F.Cu) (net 7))
 (segment (start 111.887 94.748666) (end 111.887 94.695) (width 0.4) (layer F.Cu) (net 7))
 (segment (start 114.118334 96.98) (end 111.887 94.748666) (width 0.4) (layer F.Cu) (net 7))
 (via (at 110.998 87.376) (size 1) (drill 0.5) (layers F.Cu B.Cu) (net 7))
 (segment (start 110.998 89.715073) (end 110.998 87.376) (width 0.4) (layer B.Cu) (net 7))
 (segment (start 111.887 94.695) (end 110.998 93.806) (width 0.4) (layer B.Cu) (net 7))
 (segment (start 110.998 93.806) (end 110.998 89.715073) (width 0.4) (layer B.Cu) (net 7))
 (segment (start 110.998 87.376) (end 103.885996 87.376) (width 0.4) (layer F.Cu) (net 7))
 (segment (start 100.012498 83.539888) (end 100.012498 83.502502) (width 0.4) (layer F.Cu) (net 7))
 (segment (start 99.078693 84.473693) (end 100.012498 83.539888) (width 0.4) (layer F.Cu) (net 7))
 (segment (start 103.885996 87.376) (end 100.012498 83.502502) (width 0.4) (layer F.Cu) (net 7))
 (segment (start 94.161663 77.651667) (end 96.274001 79.764005) (width 0.4) (layer B.Cu) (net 7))
 (via (at 96.774 80.264004) (size 1) (drill 0.5) (layers F.Cu B.Cu) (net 7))
 (segment (start 96.274001 79.764005) (end 96.774 80.264004) (width 0.4) (layer B.Cu) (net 7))
 (segment (start 85.271666 78.975) (end 86.594999 77.651667) (width 0.4) (layer B.Cu) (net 7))
 (segment (start 86.594999 77.651667) (end 94.161663 77.651667) (width 0.4) (layer B.Cu) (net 7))
 (segment (start 84.455 78.975) (end 85.271666 78.975) (width 0.4) (layer B.Cu) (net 7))
 (segment (start 100.012498 83.502502) (end 97.273999 80.764003) (width 0.4) (layer F.Cu) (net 7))
 (segment (start 97.273999 80.764003) (end 96.774 80.264004) (width 0.4) (layer F.Cu) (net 7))
 (segment (start 108.077 88.773) (end 108.077 93.472) (width 0.4) (layer B.Cu) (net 2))
 (segment (start 98.591384 83.185) (end 102.489 83.185) (width 0.4) (layer B.Cu) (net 2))
 (segment (start 97.829384 83.947) (end 98.591384 83.185) (width 0.4) (layer B.Cu) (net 2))
 (segment (start 89.365 81.745) (end 91.567 83.947) (width 0.4) (layer B.Cu) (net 2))
 (segment (start 96.266 83.947) (end 97.829384 83.947) (width 0.4) (layer B.Cu) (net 2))
 (segment (start 84.455 81.745) (end 89.365 81.745) (width 0.4) (layer B.Cu) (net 2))
 (segment (start 102.489 83.185) (end 108.077 88.773) (width 0.4) (layer B.Cu) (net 2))
 (segment (start 91.567 83.947) (end 93.344284 83.947) (width 0.4) (layer B.Cu) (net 2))
 (segment (start 93.344284 83.947) (end 94.106284 83.185) (width 0.4) (layer B.Cu) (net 2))
 (segment (start 94.106284 83.185) (end 95.504 83.185) (width 0.4) (layer B.Cu) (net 2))
 (segment (start 95.504 83.185) (end 96.266 83.947) (width 0.4) (layer B.Cu) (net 2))
 (segment (start 100.838 87.229592) (end 100.838 86.233) (width 0.4) (layer B.Cu) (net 6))
 (segment (start 97.981817 90.085775) (end 100.838 87.229592) (width 0.4) (layer B.Cu) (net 6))
 (segment (start 97.981817 94.677183) (end 97.981817 90.085775) (width 0.4) (layer B.Cu) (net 6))
 (segment (start 86.674 84.515) (end 91.059 88.9) (width 0.4) (layer B.Cu) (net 6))
 (segment (start 84.455 84.515) (end 86.674 84.515) (width 0.4) (layer B.Cu) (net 6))
 (segment (start 91.059 88.9) (end 91.059 92.71) (width 0.4) (layer B.Cu) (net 6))
 (segment (start 94.996 96.647) (end 96.012 96.647) (width 0.4) (layer B.Cu) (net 6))
 (segment (start 91.059 92.71) (end 94.996 96.647) (width 0.4) (layer B.Cu) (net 6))
 (segment (start 96.012 96.647) (end 97.981817 94.677183) (width 0.4) (layer B.Cu) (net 6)))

